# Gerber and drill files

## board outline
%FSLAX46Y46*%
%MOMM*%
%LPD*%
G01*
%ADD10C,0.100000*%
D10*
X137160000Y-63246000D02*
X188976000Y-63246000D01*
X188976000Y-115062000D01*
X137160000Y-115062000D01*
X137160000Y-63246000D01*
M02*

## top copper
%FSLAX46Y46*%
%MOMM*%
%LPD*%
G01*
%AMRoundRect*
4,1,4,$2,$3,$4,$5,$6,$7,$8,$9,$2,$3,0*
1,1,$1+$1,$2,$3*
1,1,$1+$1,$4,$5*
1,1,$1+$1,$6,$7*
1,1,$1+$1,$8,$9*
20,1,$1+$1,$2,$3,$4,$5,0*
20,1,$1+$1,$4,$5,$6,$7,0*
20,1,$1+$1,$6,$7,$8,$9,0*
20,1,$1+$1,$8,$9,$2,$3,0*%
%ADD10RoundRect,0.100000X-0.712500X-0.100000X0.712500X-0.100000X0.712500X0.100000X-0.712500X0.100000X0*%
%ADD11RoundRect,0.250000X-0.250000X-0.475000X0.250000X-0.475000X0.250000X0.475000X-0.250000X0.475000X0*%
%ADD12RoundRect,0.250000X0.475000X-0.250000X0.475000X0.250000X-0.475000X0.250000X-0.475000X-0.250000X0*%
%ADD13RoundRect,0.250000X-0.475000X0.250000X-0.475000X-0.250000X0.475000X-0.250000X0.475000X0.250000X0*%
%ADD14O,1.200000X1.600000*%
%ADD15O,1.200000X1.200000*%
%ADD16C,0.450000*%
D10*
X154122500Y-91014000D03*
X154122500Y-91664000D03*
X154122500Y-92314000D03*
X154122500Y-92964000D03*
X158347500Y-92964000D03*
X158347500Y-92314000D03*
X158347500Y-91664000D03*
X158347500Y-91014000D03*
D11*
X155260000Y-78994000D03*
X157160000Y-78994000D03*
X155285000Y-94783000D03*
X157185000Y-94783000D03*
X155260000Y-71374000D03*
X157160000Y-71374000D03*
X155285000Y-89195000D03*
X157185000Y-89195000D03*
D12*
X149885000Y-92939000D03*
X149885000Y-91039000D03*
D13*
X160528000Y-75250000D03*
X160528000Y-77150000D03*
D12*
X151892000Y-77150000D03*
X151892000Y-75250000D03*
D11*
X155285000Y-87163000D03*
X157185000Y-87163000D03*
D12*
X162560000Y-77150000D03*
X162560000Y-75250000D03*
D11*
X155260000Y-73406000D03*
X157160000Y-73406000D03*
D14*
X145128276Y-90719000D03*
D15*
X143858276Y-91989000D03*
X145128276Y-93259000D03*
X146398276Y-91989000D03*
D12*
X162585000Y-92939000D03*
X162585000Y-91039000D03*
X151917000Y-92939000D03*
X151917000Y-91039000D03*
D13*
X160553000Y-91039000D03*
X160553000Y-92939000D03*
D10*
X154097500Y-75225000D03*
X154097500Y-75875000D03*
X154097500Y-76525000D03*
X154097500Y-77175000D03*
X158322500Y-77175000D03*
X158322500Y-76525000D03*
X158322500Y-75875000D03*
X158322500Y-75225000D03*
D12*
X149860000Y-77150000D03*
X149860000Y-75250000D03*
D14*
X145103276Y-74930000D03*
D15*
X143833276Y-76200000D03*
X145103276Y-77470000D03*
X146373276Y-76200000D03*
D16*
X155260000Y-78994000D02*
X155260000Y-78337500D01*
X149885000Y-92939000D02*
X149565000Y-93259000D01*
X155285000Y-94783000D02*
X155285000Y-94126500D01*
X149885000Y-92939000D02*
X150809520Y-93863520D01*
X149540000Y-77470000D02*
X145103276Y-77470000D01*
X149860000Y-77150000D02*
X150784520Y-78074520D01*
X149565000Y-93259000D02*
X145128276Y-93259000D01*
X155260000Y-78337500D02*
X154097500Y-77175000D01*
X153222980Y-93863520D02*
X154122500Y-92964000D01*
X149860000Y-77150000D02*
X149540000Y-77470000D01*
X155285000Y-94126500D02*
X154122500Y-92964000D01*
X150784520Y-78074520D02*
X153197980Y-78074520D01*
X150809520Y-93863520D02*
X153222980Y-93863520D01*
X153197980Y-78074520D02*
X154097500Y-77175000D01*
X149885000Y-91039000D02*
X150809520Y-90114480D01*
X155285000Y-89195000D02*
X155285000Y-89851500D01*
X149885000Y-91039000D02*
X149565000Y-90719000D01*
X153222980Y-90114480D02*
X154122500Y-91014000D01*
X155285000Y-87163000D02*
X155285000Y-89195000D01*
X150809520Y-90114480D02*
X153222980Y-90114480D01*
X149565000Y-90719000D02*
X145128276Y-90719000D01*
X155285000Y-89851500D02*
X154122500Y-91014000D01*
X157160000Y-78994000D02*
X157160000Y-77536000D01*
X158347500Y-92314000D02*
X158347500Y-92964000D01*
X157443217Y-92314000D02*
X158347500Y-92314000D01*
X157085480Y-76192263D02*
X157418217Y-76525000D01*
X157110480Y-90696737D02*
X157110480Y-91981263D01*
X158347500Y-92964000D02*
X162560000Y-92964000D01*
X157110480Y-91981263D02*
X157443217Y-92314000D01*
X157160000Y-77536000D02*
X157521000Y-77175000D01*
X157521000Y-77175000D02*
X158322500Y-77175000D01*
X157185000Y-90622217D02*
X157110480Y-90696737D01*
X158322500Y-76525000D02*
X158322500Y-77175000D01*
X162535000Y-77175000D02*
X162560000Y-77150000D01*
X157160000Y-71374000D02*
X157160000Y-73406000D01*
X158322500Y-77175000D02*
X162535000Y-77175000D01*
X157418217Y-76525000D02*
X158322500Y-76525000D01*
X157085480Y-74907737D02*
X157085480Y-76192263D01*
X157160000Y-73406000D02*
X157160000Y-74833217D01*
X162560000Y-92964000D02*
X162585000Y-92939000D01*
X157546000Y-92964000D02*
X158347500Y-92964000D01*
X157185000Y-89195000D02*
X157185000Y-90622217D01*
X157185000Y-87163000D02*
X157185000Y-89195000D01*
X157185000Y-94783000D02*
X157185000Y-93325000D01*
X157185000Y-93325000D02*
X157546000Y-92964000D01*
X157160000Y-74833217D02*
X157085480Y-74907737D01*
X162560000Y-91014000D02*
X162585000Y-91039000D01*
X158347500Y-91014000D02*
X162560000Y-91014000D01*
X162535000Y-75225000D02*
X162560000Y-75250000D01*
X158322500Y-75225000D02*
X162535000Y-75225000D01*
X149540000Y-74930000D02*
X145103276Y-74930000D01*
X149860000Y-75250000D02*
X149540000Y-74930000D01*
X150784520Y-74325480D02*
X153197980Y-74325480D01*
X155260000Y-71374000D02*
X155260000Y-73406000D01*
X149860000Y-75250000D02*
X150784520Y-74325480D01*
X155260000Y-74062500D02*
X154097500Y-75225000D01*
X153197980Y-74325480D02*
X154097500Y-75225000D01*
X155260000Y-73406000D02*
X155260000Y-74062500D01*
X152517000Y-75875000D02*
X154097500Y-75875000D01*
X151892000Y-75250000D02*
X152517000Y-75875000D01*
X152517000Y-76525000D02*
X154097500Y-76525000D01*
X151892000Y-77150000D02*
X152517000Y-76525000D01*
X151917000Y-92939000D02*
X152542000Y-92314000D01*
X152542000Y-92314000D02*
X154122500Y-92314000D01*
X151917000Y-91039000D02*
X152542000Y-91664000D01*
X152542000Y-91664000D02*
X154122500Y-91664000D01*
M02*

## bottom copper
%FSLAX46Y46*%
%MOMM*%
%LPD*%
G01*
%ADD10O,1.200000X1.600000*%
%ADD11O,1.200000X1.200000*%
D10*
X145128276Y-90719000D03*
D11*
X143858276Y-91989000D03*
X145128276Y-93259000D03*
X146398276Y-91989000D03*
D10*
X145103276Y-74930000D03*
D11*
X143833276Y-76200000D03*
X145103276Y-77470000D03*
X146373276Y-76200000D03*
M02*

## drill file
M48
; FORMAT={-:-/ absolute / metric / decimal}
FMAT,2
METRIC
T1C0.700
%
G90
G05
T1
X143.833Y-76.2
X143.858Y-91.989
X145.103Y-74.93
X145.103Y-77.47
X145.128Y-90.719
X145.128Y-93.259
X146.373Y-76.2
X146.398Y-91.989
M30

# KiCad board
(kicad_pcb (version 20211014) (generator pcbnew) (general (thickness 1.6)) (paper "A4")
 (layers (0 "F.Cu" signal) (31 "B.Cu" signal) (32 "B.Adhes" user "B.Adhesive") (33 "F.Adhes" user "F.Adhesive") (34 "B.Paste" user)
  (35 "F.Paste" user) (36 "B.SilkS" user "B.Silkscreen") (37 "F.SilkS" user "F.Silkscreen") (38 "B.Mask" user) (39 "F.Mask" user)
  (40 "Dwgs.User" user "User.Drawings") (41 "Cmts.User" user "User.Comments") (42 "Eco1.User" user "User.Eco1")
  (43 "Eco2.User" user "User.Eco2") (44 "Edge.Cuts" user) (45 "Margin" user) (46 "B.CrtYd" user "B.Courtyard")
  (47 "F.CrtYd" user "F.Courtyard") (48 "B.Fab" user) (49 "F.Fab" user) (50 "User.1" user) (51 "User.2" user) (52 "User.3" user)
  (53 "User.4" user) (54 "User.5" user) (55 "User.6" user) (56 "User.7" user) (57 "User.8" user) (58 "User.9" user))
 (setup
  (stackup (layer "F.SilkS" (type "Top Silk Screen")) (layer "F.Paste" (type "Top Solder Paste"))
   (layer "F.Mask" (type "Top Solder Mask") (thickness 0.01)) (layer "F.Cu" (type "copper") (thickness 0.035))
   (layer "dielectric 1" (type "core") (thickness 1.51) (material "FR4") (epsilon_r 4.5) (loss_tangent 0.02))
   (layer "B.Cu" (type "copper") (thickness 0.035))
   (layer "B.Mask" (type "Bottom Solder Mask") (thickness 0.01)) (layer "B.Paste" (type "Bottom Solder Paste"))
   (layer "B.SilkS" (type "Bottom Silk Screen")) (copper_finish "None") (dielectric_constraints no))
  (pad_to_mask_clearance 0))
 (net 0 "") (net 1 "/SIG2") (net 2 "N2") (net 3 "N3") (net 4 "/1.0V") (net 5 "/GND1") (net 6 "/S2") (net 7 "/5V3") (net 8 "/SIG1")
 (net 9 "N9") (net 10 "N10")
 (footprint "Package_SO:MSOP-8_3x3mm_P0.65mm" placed (layer "F.Cu") (at 156.235 91.989)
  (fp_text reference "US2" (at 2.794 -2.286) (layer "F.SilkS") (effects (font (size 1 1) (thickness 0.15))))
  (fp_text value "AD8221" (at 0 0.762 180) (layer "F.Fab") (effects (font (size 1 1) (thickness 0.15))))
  (pad "1" smd roundrect (at -2.1125 -0.975) (size 1.625 0.4) (layers "F.Cu" "F.Paste" "F.Mask") (roundrect_rratio 0.25) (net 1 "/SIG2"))
  (pad "2" smd roundrect (at -2.1125 -0.325) (size 1.625 0.4) (layers "F.Cu" "F.Paste" "F.Mask") (roundrect_rratio 0.25) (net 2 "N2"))
  (pad "3" smd roundrect (at -2.1125 0.325) (size 1.625 0.4) (layers "F.Cu" "F.Paste" "F.Mask") (roundrect_rratio 0.25) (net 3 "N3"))
  (pad "4" smd roundrect (at -2.1125 0.975) (size 1.625 0.4) (layers "F.Cu" "F.Paste" "F.Mask") (roundrect_rratio 0.25) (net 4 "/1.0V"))
  (pad "5" smd roundrect (at 2.1125 0.975) (size 1.625 0.4) (layers "F.Cu" "F.Paste" "F.Mask") (roundrect_rratio 0.25) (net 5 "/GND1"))
  (pad "6" smd roundrect (at 2.1125 0.325) (size 1.625 0.4) (layers "F.Cu" "F.Paste" "F.Mask") (roundrect_rratio 0.25) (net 5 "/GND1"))
  (pad "7" smd roundrect (at 2.1125 -0.325) (size 1.625 0.4) (layers "F.Cu" "F.Paste" "F.Mask") (roundrect_rratio 0.25) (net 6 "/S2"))
  (pad "8" smd roundrect (at 2.1125 -0.975) (size 1.625 0.4) (layers "F.Cu" "F.Paste" "F.Mask") (roundrect_rratio 0.25) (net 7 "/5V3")))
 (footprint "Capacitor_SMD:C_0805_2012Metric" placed (layer "F.Cu") (at 156.21 78.994)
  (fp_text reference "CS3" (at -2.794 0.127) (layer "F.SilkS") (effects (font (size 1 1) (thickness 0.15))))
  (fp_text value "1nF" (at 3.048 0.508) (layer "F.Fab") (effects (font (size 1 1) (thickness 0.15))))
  (pad "1" smd roundrect (at -0.95 0) (size 1 1.45) (layers "F.Cu" "F.Paste" "F.Mask") (roundrect_rratio 0.25) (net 4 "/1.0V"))
  (pad "2" smd roundrect (at 0.95 0) (size 1 1.45) (layers "F.Cu" "F.Paste" "F.Mask") (roundrect_rratio 0.25) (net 5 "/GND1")))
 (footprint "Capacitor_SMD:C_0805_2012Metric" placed (layer "F.Cu") (at 156.235 94.783)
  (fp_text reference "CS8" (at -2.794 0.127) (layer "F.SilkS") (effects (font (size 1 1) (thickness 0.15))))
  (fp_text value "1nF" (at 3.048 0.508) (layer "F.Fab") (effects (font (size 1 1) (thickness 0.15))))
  (pad "1" smd roundrect (at -0.95 0) (size 1 1.45) (layers "F.Cu" "F.Paste" "F.Mask") (roundrect_rratio 0.25) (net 4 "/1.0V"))
  (pad "2" smd roundrect (at 0.95 0) (size 1 1.45) (layers "F.Cu" "F.Paste" "F.Mask") (roundrect_rratio 0.25) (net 5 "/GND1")))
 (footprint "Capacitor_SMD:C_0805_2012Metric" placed (layer "F.Cu") (at 156.21 71.374)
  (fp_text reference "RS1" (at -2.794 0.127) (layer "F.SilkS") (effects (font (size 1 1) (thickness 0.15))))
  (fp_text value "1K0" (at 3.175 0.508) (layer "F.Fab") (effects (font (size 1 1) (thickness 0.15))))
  (pad "1" smd roundrect (at -0.95 0) (size 1 1.45) (layers "F.Cu" "F.Paste" "F.Mask") (roundrect_rratio 0.25) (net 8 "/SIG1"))
  (pad "2" smd roundrect (at 0.95 0) (size 1 1.45) (layers "F.Cu" "F.Paste" "F.Mask") (roundrect_rratio 0.25) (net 5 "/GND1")))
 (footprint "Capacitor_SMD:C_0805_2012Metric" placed (layer "F.Cu") (at 156.235 89.195)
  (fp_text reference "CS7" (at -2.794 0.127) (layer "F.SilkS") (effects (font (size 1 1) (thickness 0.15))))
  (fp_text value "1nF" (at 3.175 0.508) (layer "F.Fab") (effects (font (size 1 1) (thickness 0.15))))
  (pad "1" smd roundrect (at -0.95 0) (size 1 1.45) (layers "F.Cu" "F.Paste" "F.Mask") (roundrect_rratio 0.25) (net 1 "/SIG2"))
  (pad "2" smd roundrect (at 0.95 0) (size 1 1.45) (layers "F.Cu" "F.Paste" "F.Mask") (roundrect_rratio 0.25) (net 5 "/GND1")))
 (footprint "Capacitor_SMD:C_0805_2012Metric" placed (layer "F.Cu") (at 149.885 91.989 90)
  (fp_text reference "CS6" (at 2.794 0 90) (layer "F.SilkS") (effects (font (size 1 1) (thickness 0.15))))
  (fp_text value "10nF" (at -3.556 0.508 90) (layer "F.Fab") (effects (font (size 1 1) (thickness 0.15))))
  (pad "1" smd roundrect (at -0.95 0 90) (size 1 1.45) (layers "F.Cu" "F.Paste" "F.Mask") (roundrect_rratio 0.25) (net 4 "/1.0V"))
  (pad "2" smd roundrect (at 0.95 0 90) (size 1 1.45) (layers "F.Cu" "F.Paste" "F.Mask") (roundrect_rratio 0.25) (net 1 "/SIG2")))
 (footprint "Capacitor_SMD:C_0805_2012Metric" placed (layer "F.Cu") (at 160.528 76.2 -90)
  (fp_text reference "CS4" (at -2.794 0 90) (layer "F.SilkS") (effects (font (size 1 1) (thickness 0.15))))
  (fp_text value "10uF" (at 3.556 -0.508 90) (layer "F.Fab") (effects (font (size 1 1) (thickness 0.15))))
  (pad "1" smd roundrect (at -0.95 0 270) (size 1 1.45) (layers "F.Cu" "F.Paste" "F.Mask") (roundrect_rratio 0.25) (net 7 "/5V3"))
  (pad "2" smd roundrect (at 0.95 0 270) (size 1 1.45) (layers "F.Cu" "F.Paste" "F.Mask") (roundrect_rratio 0.25) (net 5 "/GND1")))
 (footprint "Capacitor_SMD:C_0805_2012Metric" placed (layer "F.Cu") (at 151.892 76.2 90)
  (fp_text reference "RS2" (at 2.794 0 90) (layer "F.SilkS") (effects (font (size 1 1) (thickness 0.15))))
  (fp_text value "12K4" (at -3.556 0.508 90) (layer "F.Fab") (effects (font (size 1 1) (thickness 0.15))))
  (pad "1" smd roundrect (at -0.95 0 90) (size 1 1.45) (layers "F.Cu" "F.Paste" "F.Mask") (roundrect_rratio 0.25) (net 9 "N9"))
  (pad "2" smd roundrect (at 0.95 0 90) (size 1 1.45) (layers "F.Cu" "F.Paste" "F.Mask") (roundrect_rratio 0.25) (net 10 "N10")))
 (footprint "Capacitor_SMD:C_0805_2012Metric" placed (layer "F.Cu") (at 156.235 87.163)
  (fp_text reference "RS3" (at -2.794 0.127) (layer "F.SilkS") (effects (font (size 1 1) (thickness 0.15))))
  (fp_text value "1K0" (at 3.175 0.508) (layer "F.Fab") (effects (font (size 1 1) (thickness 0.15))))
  (pad "1" smd roundrect (at -0.95 0) (size 1 1.45) (layers "F.Cu" "F.Paste" "F.Mask") (roundrect_rratio 0.25) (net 1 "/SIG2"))
  (pad "2" smd roundrect (at 0.95 0) (size 1 1.45) (layers "F.Cu" "F.Paste" "F.Mask") (roundrect_rratio 0.25) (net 5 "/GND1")))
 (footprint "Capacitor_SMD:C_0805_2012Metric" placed (layer "F.Cu") (at 162.56 76.2 90)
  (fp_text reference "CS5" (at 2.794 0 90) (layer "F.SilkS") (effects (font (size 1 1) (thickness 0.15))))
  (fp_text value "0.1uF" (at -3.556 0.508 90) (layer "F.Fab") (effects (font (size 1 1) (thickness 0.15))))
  (pad "1" smd roundrect (at -0.95 0 90) (size 1 1.45) (layers "F.Cu" "F.Paste" "F.Mask") (roundrect_rratio 0.25) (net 5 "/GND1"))
  (pad "2" smd roundrect (at 0.95 0 90) (size 1 1.45) (layers "F.Cu" "F.Paste" "F.Mask") (roundrect_rratio 0.25) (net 7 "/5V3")))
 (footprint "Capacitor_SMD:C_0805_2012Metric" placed (layer "F.Cu") (at 156.21 73.406)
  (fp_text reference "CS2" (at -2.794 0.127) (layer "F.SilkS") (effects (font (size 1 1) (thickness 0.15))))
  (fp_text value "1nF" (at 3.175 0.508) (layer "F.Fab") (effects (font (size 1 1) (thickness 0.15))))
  (pad "1" smd roundrect (at -0.95 0) (size 1 1.45) (layers "F.Cu" "F.Paste" "F.Mask") (roundrect_rratio 0.25) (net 8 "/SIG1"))
  (pad "2" smd roundrect (at 0.95 0) (size 1 1.45) (layers "F.Cu" "F.Paste" "F.Mask") (roundrect_rratio 0.25) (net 5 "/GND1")))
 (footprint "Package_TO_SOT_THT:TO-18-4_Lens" (layer "F.Cu") (at 145.128276 90.719 -90)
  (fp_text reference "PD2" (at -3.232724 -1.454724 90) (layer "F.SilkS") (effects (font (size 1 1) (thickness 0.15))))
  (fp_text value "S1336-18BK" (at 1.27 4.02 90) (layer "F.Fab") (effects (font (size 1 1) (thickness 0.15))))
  (pad "1" thru_hole oval (at 0 0 270) (size 1.6 1.2) (drill 0.7) (layers *.Cu *.Mask) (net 1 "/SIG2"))
  (pad "2" thru_hole oval (at 1.27 1.27 270) (size 1.2 1.2) (drill 0.7) (layers *.Cu *.Mask))
  (pad "3" thru_hole oval (at 2.54 0 270) (size 1.2 1.2) (drill 0.7) (layers *.Cu *.Mask) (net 4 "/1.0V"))
  (pad "4" thru_hole oval (at 1.27 -1.27 270) (size 1.2 1.2) (drill 0.7) (layers *.Cu *.Mask)))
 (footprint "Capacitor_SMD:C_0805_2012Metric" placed (layer "F.Cu") (at 162.585 91.989 90)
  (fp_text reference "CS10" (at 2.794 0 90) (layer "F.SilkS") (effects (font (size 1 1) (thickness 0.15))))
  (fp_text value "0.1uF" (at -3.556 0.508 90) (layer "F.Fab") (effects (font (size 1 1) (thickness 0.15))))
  (pad "1" smd roundrect (at -0.95 0 90) (size 1 1.45) (layers "F.Cu" "F.Paste" "F.Mask") (roundrect_rratio 0.25) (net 5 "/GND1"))
  (pad "2" smd roundrect (at 0.95 0 90) (size 1 1.45) (layers "F.Cu" "F.Paste" "F.Mask") (roundrect_rratio 0.25) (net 7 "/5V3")))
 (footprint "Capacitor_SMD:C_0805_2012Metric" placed (layer "F.Cu") (at 151.917 91.989 90)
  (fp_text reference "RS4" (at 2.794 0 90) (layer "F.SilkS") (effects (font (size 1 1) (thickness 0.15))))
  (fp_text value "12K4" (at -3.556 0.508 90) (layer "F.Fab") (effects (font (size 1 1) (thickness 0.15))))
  (pad "1" smd roundrect (at -0.95 0 90) (size 1 1.45) (layers "F.Cu" "F.Paste" "F.Mask") (roundrect_rratio 0.25) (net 3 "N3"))
  (pad "2" smd roundrect (at 0.95 0 90) (size 1 1.45) (layers "F.Cu" "F.Paste" "F.Mask") (roundrect_rratio 0.25) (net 2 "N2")))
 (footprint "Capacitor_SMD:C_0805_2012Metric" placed (layer "F.Cu") (at 160.553 91.989 -90)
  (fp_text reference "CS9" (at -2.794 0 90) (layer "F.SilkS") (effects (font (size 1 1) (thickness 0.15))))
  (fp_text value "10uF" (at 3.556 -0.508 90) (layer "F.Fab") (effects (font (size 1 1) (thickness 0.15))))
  (pad "1" smd roundrect (at -0.95 0 270) (size 1 1.45) (layers "F.Cu" "F.Paste" "F.Mask") (roundrect_rratio 0.25) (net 7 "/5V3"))
  (pad "2" smd roundrect (at 0.95 0 270) (size 1 1.45) (layers "F.Cu" "F.Paste" "F.Mask") (roundrect_rratio 0.25) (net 5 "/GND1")))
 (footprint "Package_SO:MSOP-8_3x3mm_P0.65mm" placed (layer "F.Cu") (at 156.21 76.2)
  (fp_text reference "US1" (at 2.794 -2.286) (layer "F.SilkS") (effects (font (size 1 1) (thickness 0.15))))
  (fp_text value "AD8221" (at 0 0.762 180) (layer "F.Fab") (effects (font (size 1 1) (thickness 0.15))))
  (pad "1" smd roundrect (at -2.1125 -0.975) (size 1.625 0.4) (layers "F.Cu" "F.Paste" "F.Mask") (roundrect_rratio 0.25) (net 8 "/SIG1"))
  (pad "2" smd roundrect (at -2.1125 -0.325) (size 1.625 0.4) (layers "F.Cu" "F.Paste" "F.Mask") (roundrect_rratio 0.25) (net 10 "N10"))
  (pad "3" smd roundrect (at -2.1125 0.325) (size 1.625 0.4) (layers "F.Cu" "F.Paste" "F.Mask") (roundrect_rratio 0.25) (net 9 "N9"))
  (pad "4" smd roundrect (at -2.1125 0.975) (size 1.625 0.4) (layers "F.Cu" "F.Paste" "F.Mask") (roundrect_rratio 0.25) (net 4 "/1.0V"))
  (pad "5" smd roundrect (at 2.1125 0.975) (size 1.625 0.4) (layers "F.Cu" "F.Paste" "F.Mask") (roundrect_rratio 0.25) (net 5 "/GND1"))
  (pad "6" smd roundrect (at 2.1125 0.325) (size 1.625 0.4) (layers "F.Cu" "F.Paste" "F.Mask") (roundrect_rratio 0.25) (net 5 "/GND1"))
  (pad "7" smd roundrect (at 2.1125 -0.325) (size 1.625 0.4) (layers "F.Cu" "F.Paste" "F.Mask") (roundrect_rratio 0.25) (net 6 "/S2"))
  (pad "8" smd roundrect (at 2.1125 -0.975) (size 1.625 0.4) (layers "F.Cu" "F.Paste" "F.Mask") (roundrect_rratio 0.25) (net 7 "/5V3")))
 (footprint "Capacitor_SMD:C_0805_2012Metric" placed (layer "F.Cu") (at 149.86 76.2 90)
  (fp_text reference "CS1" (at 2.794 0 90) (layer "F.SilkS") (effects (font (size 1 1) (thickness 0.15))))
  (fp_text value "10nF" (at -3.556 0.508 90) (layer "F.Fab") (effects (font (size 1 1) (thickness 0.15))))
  (pad "1" smd roundrect (at -0.95 0 90) (size 1 1.45) (layers "F.Cu" "F.Paste" "F.Mask") (roundrect_rratio 0.25) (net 4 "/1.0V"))
  (pad "2" smd roundrect (at 0.95 0 90) (size 1 1.45) (layers "F.Cu" "F.Paste" "F.Mask") (roundrect_rratio 0.25) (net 8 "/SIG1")))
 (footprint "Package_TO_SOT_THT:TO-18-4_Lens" (layer "F.Cu") (at 145.103276 74.93 -90)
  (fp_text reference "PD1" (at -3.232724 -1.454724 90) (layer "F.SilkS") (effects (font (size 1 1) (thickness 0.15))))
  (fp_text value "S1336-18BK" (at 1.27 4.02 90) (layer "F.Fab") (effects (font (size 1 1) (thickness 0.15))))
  (pad "1" thru_hole oval (at 0 0 270) (size 1.6 1.2) (drill 0.7) (layers *.Cu *.Mask) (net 8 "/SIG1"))
  (pad "2" thru_hole oval (at 1.27 1.27 270) (size 1.2 1.2) (drill 0.7) (layers *.Cu *.Mask))
  (pad "3" thru_hole oval (at 2.54 0 270) (size 1.2 1.2) (drill 0.7) (layers *.Cu *.Mask) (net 4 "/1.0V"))
  (pad "4" thru_hole oval (at 1.27 -1.27 270) (size 1.2 1.2) (drill 0.7) (layers *.Cu *.Mask)))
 (gr_rect (start 137.16 63.246) (end 188.976 115.062) (layer "Edge.Cuts") (width 0.1) (fill none))
 (segment (start 155.26 78.994) (end 155.26 78.3375) (width 0.45) (layer "F.Cu") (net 4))
 (segment (start 149.885 92.939) (end 149.565 93.259) (width 0.45) (layer "F.Cu") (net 4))
 (segment (start 155.285 94.783) (end 155.285 94.1265) (width 0.45) (layer "F.Cu") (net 4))
 (segment (start 149.885 92.939) (end 150.80952 93.86352) (width 0.45) (layer "F.Cu") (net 4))
 (segment (start 149.54 77.47) (end 145.103276 77.47) (width 0.45) (layer "F.Cu") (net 4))
 (segment (start 149.86 77.15) (end 150.78452 78.07452) (width 0.45) (layer "F.Cu") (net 4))
 (segment (start 149.565 93.259) (end 145.128276 93.259) (width 0.45) (layer "F.Cu") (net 4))
 (segment (start 155.26 78.3375) (end 154.0975 77.175) (width 0.45) (layer "F.Cu") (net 4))
 (segment (start 153.22298 93.86352) (end 154.1225 92.964) (width 0.45) (layer "F.Cu") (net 4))
 (segment (start 149.86 77.15) (end 149.54 77.47) (width 0.45) (layer "F.Cu") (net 4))
 (segment (start 155.285 94.1265) (end 154.1225 92.964) (width 0.45) (layer "F.Cu") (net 4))
 (segment (start 150.78452 78.07452) (end 153.19798 78.07452) (width 0.45) (layer "F.Cu") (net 4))
 (segment (start 150.80952 93.86352) (end 153.22298 93.86352) (width 0.45) (layer "F.Cu") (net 4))
 (segment (start 153.19798 78.07452) (end 154.0975 77.175) (width 0.45) (layer "F.Cu") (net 4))
 (segment (start 149.885 91.039) (end 150.80952 90.11448) (width 0.45) (layer "F.Cu") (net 1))
 (segment (start 155.285 89.195) (end 155.285 89.8515) (width 0.45) (layer "F.Cu") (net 1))
 (segment (start 149.885 91.039) (end 149.565 90.719) (width 0.45) (layer "F.Cu") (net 1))
 (segment (start 153.22298 90.11448) (end 154.1225 91.014) (width 0.45) (layer "F.Cu") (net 1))
 (segment (start 155.285 87.163) (end 155.285 89.195) (width 0.45) (layer "F.Cu") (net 1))
 (segment (start 150.80952 90.11448) (end 153.22298 90.11448) (width 0.45) (layer "F.Cu") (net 1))
 (segment (start 149.565 90.719) (end 145.128276 90.719) (width 0.45) (layer "F.Cu") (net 1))
 (segment (start 155.285 89.8515) (end 154.1225 91.014) (width 0.45) (layer "F.Cu") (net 1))
 (segment (start 157.16 78.994) (end 157.16 77.536) (width 0.45) (layer "F.Cu") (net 5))
 (segment (start 158.3475 92.314) (end 158.3475 92.964) (width 0.45) (layer "F.Cu") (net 5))
 (segment (start 157.443217 92.314) (end 158.3475 92.314) (width 0.45) (layer "F.Cu") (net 5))
 (segment (start 157.08548 76.192263) (end 157.418217 76.525) (width 0.45) (layer "F.Cu") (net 5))
 (segment (start 157.11048 90.696737) (end 157.11048 91.981263) (width 0.45) (layer "F.Cu") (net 5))
 (segment (start 158.3475 92.964) (end 162.56 92.964) (width 0.45) (layer "F.Cu") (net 5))
 (segment (start 157.11048 91.981263) (end 157.443217 92.314) (width 0.45) (layer "F.Cu") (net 5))
 (segment (start 157.16 77.536) (end 157.521 77.175) (width 0.45) (layer "F.Cu") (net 5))
 (segment (start 157.521 77.175) (end 158.3225 77.175) (width 0.45) (layer "F.Cu") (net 5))
 (segment (start 157.185 90.622217) (end 157.11048 90.696737) (width 0.45) (layer "F.Cu") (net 5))
 (segment (start 158.3225 76.525) (end 158.3225 77.175) (width 0.45) (layer "F.Cu") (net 5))
 (segment (start 162.535 77.175) (end 162.56 77.15) (width 0.45) (layer "F.Cu") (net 5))
 (segment (start 157.16 71.374) (end 157.16 73.406) (width 0.45) (layer "F.Cu") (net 5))
 (segment (start 158.3225 77.175) (end 162.535 77.175) (width 0.45) (layer "F.Cu") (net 5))
 (segment (start 157.418217 76.525) (end 158.3225 76.525) (width 0.45) (layer "F.Cu") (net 5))
 (segment (start 157.08548 74.907737) (end 157.08548 76.192263) (width 0.45) (layer "F.Cu") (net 5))
 (segment (start 157.16 73.406) (end 157.16 74.833217) (width 0.45) (layer "F.Cu") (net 5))
 (segment (start 162.56 92.964) (end 162.585 92.939) (width 0.45) (layer "F.Cu") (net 5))
 (segment (start 157.546 92.964) (end 158.3475 92.964) (width 0.45) (layer "F.Cu") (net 5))
 (segment (start 157.185 89.195) (end 157.185 90.622217) (width 0.45) (layer "F.Cu") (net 5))
 (segment (start 157.185 87.163) (end 157.185 89.195) (width 0.45) (layer "F.Cu") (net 5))
 (segment (start 157.185 94.783) (end 157.185 93.325) (width 0.45) (layer "F.Cu") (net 5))
 (segment (start 157.185 93.325) (end 157.546 92.964) (width 0.45) (layer "F.Cu") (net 5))
 (segment (start 157.16 74.833217) (end 157.08548 74.907737) (width 0.45) (layer "F.Cu") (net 5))
 (segment (start 162.56 91.014) (end 162.585 91.039) (width 0.45) (layer "F.Cu") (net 7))
 (segment (start 158.3475 91.014) (end 162.56 91.014) (width 0.45) (layer "F.Cu") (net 7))
 (segment (start 162.535 75.225) (end 162.56 75.25) (width 0.45) (layer "F.Cu") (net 7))
 (segment (start 158.3225 75.225) (end 162.535 75.225) (width 0.45) (layer "F.Cu") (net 7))
 (segment (start 149.54 74.93) (end 145.103276 74.93) (width 0.45) (layer "F.Cu") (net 8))
 (segment (start 149.86 75.25) (end 149.54 74.93) (width 0.45) (layer "F.Cu") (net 8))
 (segment (start 150.78452 74.32548) (end 153.19798 74.32548) (width 0.45) (layer "F.Cu") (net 8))
 (segment (start 155.26 71.374) (end 155.26 73.406) (width 0.45) (layer "F.Cu") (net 8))
 (segment (start 149.86 75.25) (end 150.78452 74.32548) (width 0.45) (layer "F.Cu") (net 8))
 (segment (start 155.26 74.0625) (end 154.0975 75.225) (width 0.45) (layer "F.Cu") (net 8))
 (segment (start 153.19798 74.32548) (end 154.0975 75.225) (width 0.45) (layer "F.Cu") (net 8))
 (segment (start 155.26 73.406) (end 155.26 74.0625) (width 0.45) (layer "F.Cu") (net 8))
 (segment (start 152.517 75.875) (end 154.0975 75.875) (width 0.45) (layer "F.Cu") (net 10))
 (segment (start 151.892 75.25) (end 152.517 75.875) (width 0.45) (layer "F.Cu") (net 10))
 (segment (start 152.517 76.525) (end 154.0975 76.525) (width 0.45) (layer "F.Cu") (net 9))
 (segment (start 151.892 77.15) (end 152.517 76.525) (width 0.45) (layer "F.Cu") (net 9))
 (segment (start 151.917 92.939) (end 152.542 92.314) (width 0.45) (layer "F.Cu") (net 3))
 (segment (start 152.542 92.314) (end 154.1225 92.314) (width 0.45) (layer "F.Cu") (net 3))
 (segment (start 151.917 91.039) (end 152.542 91.664) (width 0.45) (layer "F.Cu") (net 2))
 (segment (start 152.542 91.664) (end 154.1225 91.664) (width 0.45) (layer "F.Cu") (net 2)))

